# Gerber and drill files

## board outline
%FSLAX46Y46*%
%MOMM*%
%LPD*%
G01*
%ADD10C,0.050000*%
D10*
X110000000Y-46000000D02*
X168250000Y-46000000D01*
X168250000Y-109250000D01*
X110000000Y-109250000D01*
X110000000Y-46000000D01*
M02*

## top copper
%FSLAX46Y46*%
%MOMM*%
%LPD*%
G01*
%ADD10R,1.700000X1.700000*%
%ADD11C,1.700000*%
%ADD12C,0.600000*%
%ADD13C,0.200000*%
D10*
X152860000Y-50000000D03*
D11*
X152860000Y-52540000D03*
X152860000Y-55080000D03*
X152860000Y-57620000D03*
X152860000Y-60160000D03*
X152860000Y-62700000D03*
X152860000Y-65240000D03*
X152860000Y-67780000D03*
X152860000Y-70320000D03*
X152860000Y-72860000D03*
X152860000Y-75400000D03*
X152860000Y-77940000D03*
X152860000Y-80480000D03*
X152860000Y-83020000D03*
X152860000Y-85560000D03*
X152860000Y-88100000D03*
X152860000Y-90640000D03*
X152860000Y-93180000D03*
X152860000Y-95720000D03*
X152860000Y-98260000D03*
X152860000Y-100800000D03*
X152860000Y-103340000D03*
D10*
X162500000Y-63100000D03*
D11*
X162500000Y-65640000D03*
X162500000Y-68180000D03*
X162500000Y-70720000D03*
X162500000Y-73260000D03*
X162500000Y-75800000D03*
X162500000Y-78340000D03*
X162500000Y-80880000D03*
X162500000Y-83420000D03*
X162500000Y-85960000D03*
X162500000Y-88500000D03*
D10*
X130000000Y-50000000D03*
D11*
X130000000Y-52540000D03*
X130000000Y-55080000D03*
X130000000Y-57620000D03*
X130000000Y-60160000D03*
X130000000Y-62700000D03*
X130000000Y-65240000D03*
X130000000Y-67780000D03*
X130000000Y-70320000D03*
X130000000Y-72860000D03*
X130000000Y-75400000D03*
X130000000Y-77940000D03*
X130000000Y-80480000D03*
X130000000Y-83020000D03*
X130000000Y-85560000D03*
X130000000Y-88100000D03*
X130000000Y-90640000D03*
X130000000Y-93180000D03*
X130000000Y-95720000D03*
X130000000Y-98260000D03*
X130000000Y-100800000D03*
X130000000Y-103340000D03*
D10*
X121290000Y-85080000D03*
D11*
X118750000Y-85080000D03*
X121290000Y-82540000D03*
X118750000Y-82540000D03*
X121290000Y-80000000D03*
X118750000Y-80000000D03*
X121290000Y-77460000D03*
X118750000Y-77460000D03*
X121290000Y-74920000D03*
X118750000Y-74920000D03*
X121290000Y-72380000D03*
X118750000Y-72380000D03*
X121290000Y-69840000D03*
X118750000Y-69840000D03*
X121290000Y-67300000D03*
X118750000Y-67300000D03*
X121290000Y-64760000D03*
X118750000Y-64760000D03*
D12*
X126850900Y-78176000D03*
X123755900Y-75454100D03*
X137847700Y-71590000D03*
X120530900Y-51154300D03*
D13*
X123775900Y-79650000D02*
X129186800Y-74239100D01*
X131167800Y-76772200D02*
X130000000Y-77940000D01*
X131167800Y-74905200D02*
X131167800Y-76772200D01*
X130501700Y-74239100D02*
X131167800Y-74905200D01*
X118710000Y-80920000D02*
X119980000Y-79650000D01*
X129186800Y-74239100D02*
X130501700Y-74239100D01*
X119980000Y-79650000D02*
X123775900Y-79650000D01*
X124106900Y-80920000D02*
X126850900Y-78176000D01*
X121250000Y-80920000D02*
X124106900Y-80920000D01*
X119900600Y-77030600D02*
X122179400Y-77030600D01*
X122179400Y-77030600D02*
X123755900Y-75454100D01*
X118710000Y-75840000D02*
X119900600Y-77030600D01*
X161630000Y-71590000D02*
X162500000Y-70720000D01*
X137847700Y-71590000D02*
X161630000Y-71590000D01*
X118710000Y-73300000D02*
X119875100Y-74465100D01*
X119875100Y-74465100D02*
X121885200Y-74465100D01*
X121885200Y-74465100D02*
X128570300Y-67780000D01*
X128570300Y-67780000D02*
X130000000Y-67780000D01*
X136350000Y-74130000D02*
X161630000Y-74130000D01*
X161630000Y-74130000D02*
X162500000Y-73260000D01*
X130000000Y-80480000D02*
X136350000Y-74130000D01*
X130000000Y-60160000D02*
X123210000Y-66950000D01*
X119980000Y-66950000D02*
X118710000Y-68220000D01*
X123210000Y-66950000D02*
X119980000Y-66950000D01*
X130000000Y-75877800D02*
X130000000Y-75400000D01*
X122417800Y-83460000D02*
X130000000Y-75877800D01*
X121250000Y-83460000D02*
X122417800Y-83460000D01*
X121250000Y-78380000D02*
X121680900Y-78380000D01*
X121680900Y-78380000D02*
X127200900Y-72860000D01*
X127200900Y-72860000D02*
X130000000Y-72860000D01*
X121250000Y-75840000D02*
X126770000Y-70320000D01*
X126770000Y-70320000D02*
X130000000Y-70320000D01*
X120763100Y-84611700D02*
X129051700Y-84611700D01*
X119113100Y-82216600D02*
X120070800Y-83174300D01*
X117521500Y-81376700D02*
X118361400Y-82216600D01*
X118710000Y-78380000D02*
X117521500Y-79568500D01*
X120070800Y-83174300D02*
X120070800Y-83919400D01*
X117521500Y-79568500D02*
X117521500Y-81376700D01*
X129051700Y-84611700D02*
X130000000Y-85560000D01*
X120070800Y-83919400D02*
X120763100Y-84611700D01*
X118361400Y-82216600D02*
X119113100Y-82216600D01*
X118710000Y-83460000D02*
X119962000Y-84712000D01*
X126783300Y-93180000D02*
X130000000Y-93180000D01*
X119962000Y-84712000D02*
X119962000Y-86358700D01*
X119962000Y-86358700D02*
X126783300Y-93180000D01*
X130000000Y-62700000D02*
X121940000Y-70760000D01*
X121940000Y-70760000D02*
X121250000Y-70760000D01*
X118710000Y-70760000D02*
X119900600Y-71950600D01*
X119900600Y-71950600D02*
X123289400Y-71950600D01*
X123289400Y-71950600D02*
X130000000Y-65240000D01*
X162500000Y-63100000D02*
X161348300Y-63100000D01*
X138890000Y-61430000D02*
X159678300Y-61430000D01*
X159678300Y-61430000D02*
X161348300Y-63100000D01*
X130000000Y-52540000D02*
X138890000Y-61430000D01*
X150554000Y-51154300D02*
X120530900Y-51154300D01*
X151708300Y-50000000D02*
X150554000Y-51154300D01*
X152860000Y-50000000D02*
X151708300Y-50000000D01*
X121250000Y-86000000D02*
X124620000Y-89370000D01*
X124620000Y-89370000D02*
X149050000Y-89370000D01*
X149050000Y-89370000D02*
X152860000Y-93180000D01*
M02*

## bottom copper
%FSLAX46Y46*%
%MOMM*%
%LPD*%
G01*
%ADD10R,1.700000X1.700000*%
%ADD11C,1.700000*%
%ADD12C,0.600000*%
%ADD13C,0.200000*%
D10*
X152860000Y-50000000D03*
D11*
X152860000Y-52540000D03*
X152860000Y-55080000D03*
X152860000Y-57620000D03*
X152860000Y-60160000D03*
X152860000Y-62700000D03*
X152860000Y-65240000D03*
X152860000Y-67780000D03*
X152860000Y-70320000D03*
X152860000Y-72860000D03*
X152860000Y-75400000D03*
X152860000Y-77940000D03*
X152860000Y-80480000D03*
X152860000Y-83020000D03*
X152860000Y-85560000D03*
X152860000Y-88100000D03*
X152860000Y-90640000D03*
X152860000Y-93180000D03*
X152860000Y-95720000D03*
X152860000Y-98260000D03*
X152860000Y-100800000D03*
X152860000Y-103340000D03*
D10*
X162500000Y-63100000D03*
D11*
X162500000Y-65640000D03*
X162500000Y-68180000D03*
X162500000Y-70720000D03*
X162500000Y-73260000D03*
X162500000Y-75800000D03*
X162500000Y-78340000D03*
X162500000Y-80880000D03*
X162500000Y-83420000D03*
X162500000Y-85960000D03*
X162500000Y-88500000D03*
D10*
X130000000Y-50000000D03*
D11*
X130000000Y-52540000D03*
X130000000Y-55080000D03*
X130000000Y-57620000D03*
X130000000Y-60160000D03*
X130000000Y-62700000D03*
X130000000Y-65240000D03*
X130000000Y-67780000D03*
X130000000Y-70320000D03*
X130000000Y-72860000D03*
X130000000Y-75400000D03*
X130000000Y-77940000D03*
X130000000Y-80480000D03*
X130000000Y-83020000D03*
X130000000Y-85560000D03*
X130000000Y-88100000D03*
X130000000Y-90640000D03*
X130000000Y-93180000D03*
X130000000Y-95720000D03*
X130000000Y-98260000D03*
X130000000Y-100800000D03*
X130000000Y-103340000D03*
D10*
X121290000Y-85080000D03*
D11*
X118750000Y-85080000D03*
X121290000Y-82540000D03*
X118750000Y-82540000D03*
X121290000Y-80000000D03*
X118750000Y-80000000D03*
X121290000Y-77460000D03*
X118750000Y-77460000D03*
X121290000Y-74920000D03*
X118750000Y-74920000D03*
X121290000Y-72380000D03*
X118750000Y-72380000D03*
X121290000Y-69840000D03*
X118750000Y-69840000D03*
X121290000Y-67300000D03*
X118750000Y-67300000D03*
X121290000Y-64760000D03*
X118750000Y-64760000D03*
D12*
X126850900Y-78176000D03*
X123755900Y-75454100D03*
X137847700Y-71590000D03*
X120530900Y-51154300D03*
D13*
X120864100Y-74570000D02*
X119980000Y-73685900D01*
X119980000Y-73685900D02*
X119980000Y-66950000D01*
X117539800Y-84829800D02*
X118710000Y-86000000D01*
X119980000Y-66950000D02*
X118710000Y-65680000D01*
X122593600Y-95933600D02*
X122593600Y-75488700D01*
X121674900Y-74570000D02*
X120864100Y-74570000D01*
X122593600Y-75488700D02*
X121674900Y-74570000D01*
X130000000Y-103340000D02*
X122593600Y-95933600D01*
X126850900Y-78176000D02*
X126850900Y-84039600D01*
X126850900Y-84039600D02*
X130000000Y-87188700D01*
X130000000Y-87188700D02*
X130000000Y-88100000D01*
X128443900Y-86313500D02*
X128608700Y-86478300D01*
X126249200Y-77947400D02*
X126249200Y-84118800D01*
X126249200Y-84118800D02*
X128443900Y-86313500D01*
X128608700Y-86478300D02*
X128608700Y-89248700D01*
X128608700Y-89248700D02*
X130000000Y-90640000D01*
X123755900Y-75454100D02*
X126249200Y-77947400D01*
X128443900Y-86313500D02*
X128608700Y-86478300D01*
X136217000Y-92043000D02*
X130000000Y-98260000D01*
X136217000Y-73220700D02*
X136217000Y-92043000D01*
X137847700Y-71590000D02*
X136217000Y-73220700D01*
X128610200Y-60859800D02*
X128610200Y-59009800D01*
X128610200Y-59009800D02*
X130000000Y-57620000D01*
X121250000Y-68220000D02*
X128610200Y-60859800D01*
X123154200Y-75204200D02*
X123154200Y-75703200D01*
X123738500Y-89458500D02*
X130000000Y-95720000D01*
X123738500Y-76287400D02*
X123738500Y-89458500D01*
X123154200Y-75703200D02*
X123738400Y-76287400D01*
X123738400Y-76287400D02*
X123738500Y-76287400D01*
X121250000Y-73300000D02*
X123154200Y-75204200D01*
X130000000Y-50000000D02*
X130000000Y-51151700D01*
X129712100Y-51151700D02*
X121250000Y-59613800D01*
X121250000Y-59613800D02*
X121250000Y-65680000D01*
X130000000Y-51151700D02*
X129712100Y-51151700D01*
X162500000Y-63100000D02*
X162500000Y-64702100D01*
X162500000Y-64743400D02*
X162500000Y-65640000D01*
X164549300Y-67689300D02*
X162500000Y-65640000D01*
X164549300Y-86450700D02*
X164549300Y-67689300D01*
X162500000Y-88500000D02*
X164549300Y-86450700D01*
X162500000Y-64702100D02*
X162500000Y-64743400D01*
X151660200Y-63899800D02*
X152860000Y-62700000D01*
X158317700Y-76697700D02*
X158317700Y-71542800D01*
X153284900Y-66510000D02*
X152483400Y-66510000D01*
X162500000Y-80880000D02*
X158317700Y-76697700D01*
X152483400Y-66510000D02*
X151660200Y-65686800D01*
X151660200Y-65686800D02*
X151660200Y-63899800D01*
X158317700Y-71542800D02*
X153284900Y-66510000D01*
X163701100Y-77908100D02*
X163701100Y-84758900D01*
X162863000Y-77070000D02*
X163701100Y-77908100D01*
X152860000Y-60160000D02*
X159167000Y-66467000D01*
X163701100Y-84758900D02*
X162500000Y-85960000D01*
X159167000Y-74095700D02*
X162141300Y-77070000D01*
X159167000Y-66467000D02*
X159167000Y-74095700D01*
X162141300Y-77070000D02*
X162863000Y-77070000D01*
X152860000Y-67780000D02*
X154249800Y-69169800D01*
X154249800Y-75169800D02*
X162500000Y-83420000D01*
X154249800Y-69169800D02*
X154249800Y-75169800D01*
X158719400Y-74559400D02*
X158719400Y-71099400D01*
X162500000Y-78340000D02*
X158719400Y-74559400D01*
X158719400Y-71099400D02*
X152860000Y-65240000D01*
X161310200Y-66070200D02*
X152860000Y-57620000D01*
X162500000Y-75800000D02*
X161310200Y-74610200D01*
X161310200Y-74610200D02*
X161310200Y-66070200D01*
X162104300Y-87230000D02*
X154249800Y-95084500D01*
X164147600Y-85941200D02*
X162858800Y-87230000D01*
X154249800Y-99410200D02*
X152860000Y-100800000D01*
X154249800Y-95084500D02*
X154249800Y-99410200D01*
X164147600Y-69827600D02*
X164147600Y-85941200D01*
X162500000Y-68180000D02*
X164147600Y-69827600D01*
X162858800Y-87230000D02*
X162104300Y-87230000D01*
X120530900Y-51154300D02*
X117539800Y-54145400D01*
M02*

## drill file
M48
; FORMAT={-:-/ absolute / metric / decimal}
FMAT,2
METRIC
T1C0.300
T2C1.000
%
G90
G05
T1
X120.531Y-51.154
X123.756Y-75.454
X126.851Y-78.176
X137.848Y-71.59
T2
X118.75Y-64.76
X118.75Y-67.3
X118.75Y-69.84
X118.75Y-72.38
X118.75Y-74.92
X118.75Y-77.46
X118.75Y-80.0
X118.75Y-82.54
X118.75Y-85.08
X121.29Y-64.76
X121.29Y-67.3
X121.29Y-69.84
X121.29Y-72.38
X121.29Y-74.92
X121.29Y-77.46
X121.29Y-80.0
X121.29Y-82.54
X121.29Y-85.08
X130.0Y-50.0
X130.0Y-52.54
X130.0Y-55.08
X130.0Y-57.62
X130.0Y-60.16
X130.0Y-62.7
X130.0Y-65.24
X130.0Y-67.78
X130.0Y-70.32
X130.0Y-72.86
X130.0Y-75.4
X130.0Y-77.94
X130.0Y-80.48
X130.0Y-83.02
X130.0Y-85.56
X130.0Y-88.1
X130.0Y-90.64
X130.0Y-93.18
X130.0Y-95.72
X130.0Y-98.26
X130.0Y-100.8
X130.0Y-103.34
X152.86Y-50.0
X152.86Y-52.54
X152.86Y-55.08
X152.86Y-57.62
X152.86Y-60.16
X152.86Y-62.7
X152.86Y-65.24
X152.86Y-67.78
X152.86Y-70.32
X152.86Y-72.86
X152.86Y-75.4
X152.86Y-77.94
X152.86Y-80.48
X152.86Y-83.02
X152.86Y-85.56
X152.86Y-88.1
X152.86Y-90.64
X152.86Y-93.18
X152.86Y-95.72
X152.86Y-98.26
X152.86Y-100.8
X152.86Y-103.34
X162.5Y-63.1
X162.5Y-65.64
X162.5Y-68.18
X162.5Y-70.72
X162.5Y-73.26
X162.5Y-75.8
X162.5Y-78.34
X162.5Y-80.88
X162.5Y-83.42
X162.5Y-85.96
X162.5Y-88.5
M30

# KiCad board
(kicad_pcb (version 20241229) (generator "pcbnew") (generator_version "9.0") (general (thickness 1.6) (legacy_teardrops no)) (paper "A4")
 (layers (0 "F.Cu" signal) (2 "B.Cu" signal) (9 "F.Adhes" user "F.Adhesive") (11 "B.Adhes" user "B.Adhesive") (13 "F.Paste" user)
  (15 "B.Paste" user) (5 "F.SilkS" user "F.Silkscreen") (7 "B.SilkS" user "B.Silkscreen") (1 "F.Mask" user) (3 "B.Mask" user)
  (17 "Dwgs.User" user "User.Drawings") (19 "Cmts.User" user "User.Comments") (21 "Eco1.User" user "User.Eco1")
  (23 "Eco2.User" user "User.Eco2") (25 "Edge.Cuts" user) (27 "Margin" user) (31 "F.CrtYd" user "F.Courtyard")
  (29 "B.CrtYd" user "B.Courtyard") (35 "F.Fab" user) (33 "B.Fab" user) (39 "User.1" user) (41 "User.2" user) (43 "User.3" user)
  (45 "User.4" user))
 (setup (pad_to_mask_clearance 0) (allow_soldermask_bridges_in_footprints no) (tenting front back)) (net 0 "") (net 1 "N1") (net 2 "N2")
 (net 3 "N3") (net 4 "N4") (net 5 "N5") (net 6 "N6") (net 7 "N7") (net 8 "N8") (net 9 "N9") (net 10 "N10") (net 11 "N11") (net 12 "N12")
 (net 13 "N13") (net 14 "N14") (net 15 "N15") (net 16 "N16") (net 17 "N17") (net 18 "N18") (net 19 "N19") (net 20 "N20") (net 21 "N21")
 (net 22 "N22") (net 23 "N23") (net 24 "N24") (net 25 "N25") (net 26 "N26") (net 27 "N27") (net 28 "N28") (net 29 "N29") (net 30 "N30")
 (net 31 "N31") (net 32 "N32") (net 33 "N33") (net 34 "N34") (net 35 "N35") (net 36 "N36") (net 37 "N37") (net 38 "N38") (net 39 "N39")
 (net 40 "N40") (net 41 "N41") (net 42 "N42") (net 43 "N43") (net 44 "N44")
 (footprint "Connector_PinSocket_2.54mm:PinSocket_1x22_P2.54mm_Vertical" (layer "F.Cu") (at 152.86 50)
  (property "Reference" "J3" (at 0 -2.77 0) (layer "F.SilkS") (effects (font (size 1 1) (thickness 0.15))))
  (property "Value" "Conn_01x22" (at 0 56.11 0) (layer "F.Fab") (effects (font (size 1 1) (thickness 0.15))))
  (pad "1" thru_hole rect (at 0 0) (size 1.7 1.7) (drill 1) (layers "*.Cu" "*.Mask") (remove_unused_layers no) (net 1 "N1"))
  (pad "2" thru_hole circle (at 0 2.54) (size 1.7 1.7) (drill 1) (layers "*.Cu" "*.Mask") (remove_unused_layers no) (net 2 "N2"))
  (pad "3" thru_hole circle (at 0 5.08) (size 1.7 1.7) (drill 1) (layers "*.Cu" "*.Mask") (remove_unused_layers no) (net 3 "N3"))
  (pad "4" thru_hole circle (at 0 7.62) (size 1.7 1.7) (drill 1) (layers "*.Cu" "*.Mask") (remove_unused_layers no) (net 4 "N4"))
  (pad "5" thru_hole circle (at 0 10.16) (size 1.7 1.7) (drill 1) (layers "*.Cu" "*.Mask") (remove_unused_layers no) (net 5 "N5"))
  (pad "6" thru_hole circle (at 0 12.7) (size 1.7 1.7) (drill 1) (layers "*.Cu" "*.Mask") (remove_unused_layers no) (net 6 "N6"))
  (pad "7" thru_hole circle (at 0 15.24) (size 1.7 1.7) (drill 1) (layers "*.Cu" "*.Mask") (remove_unused_layers no) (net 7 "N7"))
  (pad "8" thru_hole circle (at 0 17.78) (size 1.7 1.7) (drill 1) (layers "*.Cu" "*.Mask") (remove_unused_layers no) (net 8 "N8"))
  (pad "9" thru_hole circle (at 0 20.32) (size 1.7 1.7) (drill 1) (layers "*.Cu" "*.Mask") (remove_unused_layers no) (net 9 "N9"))
  (pad "10" thru_hole circle (at 0 22.86) (size 1.7 1.7) (drill 1) (layers "*.Cu" "*.Mask") (remove_unused_layers no) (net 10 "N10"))
  (pad "11" thru_hole circle (at 0 25.4) (size 1.7 1.7) (drill 1) (layers "*.Cu" "*.Mask") (remove_unused_layers no) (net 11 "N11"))
  (pad "12" thru_hole circle (at 0 27.94) (size 1.7 1.7) (drill 1) (layers "*.Cu" "*.Mask") (remove_unused_layers no) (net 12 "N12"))
  (pad "13" thru_hole circle (at 0 30.48) (size 1.7 1.7) (drill 1) (layers "*.Cu" "*.Mask") (remove_unused_layers no) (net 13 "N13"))
  (pad "14" thru_hole circle (at 0 33.02) (size 1.7 1.7) (drill 1) (layers "*.Cu" "*.Mask") (remove_unused_layers no) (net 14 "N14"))
  (pad "15" thru_hole circle (at 0 35.56) (size 1.7 1.7) (drill 1) (layers "*.Cu" "*.Mask") (remove_unused_layers no) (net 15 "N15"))
  (pad "16" thru_hole circle (at 0 38.1) (size 1.7 1.7) (drill 1) (layers "*.Cu" "*.Mask") (remove_unused_layers no) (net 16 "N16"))
  (pad "17" thru_hole circle (at 0 40.64) (size 1.7 1.7) (drill 1) (layers "*.Cu" "*.Mask") (remove_unused_layers no) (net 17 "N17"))
  (pad "18" thru_hole circle (at 0 43.18) (size 1.7 1.7) (drill 1) (layers "*.Cu" "*.Mask") (remove_unused_layers no) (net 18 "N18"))
  (pad "19" thru_hole circle (at 0 45.72) (size 1.7 1.7) (drill 1) (layers "*.Cu" "*.Mask") (remove_unused_layers no) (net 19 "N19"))
  (pad "20" thru_hole circle (at 0 48.26) (size 1.7 1.7) (drill 1) (layers "*.Cu" "*.Mask") (remove_unused_layers no) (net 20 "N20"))
  (pad "21" thru_hole circle (at 0 50.8) (size 1.7 1.7) (drill 1) (layers "*.Cu" "*.Mask") (remove_unused_layers no) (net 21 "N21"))
  (pad "22" thru_hole circle (at 0 53.34) (size 1.7 1.7) (drill 1) (layers "*.Cu" "*.Mask") (remove_unused_layers no) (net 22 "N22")))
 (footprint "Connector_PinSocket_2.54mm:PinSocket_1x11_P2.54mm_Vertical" (layer "F.Cu") (at 162.5 63.1)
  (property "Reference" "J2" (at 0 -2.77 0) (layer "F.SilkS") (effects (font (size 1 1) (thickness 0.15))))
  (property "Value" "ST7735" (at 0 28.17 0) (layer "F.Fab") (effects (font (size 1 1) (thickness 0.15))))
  (pad "1" thru_hole rect (at 0 0) (size 1.7 1.7) (drill 1) (layers "*.Cu" "*.Mask") (remove_unused_layers no) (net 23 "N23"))
  (pad "2" thru_hole circle (at 0 2.54) (size 1.7 1.7) (drill 1) (layers "*.Cu" "*.Mask") (remove_unused_layers no) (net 23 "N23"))
  (pad "3" thru_hole circle (at 0 5.08) (size 1.7 1.7) (drill 1) (layers "*.Cu" "*.Mask") (remove_unused_layers no) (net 21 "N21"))
  (pad "4" thru_hole circle (at 0 7.62) (size 1.7 1.7) (drill 1) (layers "*.Cu" "*.Mask") (remove_unused_layers no) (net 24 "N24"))
  (pad "5" thru_hole circle (at 0 10.16) (size 1.7 1.7) (drill 1) (layers "*.Cu" "*.Mask") (remove_unused_layers no) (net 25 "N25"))
  (pad "6" thru_hole circle (at 0 12.7) (size 1.7 1.7) (drill 1) (layers "*.Cu" "*.Mask") (remove_unused_layers no) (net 4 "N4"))
  (pad "7" thru_hole circle (at 0 15.24) (size 1.7 1.7) (drill 1) (layers "*.Cu" "*.Mask") (remove_unused_layers no) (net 7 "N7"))
  (pad "8" thru_hole circle (at 0 17.78) (size 1.7 1.7) (drill 1) (layers "*.Cu" "*.Mask") (remove_unused_layers no) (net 6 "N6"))
  (pad "9" thru_hole circle (at 0 20.32) (size 1.7 1.7) (drill 1) (layers "*.Cu" "*.Mask") (remove_unused_layers no) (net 8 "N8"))
  (pad "10" thru_hole circle (at 0 22.86) (size 1.7 1.7) (drill 1) (layers "*.Cu" "*.Mask") (remove_unused_layers no) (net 5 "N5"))
  (pad "11" thru_hole circle (at 0 25.4) (size 1.7 1.7) (drill 1) (layers "*.Cu" "*.Mask") (remove_unused_layers no) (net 23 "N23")))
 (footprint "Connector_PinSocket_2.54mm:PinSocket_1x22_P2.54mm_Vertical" (layer "F.Cu") (at 130 50)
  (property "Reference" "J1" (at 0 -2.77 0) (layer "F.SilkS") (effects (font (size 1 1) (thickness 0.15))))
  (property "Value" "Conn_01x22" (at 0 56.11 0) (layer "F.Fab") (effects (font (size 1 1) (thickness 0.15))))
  (pad "1" thru_hole rect (at 0 0) (size 1.7 1.7) (drill 1) (layers "*.Cu" "*.Mask") (remove_unused_layers no) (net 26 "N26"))
  (pad "2" thru_hole circle (at 0 2.54) (size 1.7 1.7) (drill 1) (layers "*.Cu" "*.Mask") (remove_unused_layers no) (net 23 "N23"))
  (pad "3" thru_hole circle (at 0 5.08) (size 1.7 1.7) (drill 1) (layers "*.Cu" "*.Mask") (remove_unused_layers no) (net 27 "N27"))
  (pad "4" thru_hole circle (at 0 7.62) (size 1.7 1.7) (drill 1) (layers "*.Cu" "*.Mask") (remove_unused_layers no) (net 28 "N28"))
  (pad "5" thru_hole circle (at 0 10.16) (size 1.7 1.7) (drill 1) (layers "*.Cu" "*.Mask") (remove_unused_layers no) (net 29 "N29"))
  (pad "6" thru_hole circle (at 0 12.7) (size 1.7 1.7) (drill 1) (layers "*.Cu" "*.Mask") (remove_unused_layers no) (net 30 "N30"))
  (pad "7" thru_hole circle (at 0 15.24) (size 1.7 1.7) (drill 1) (layers "*.Cu" "*.Mask") (remove_unused_layers no) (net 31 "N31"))
  (pad "8" thru_hole circle (at 0 17.78) (size 1.7 1.7) (drill 1) (layers "*.Cu" "*.Mask") (remove_unused_layers no) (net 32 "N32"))
  (pad "9" thru_hole circle (at 0 20.32) (size 1.7 1.7) (drill 1) (layers "*.Cu" "*.Mask") (remove_unused_layers no) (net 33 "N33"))
  (pad "10" thru_hole circle (at 0 22.86) (size 1.7 1.7) (drill 1) (layers "*.Cu" "*.Mask") (remove_unused_layers no) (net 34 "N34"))
  (pad "11" thru_hole circle (at 0 25.4) (size 1.7 1.7) (drill 1) (layers "*.Cu" "*.Mask") (remove_unused_layers no) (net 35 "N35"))
  (pad "12" thru_hole circle (at 0 27.94) (size 1.7 1.7) (drill 1) (layers "*.Cu" "*.Mask") (remove_unused_layers no) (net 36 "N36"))
  (pad "13" thru_hole circle (at 0 30.48) (size 1.7 1.7) (drill 1) (layers "*.Cu" "*.Mask") (remove_unused_layers no) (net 25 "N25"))
  (pad "14" thru_hole circle (at 0 33.02) (size 1.7 1.7) (drill 1) (layers "*.Cu" "*.Mask") (remove_unused_layers no) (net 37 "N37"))
  (pad "15" thru_hole circle (at 0 35.56) (size 1.7 1.7) (drill 1) (layers "*.Cu" "*.Mask") (remove_unused_layers no) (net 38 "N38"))
  (pad "16" thru_hole circle (at 0 38.1) (size 1.7 1.7) (drill 1) (layers "*.Cu" "*.Mask") (remove_unused_layers no) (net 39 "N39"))
  (pad "17" thru_hole circle (at 0 40.64) (size 1.7 1.7) (drill 1) (layers "*.Cu" "*.Mask") (remove_unused_layers no) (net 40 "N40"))
  (pad "18" thru_hole circle (at 0 43.18) (size 1.7 1.7) (drill 1) (layers "*.Cu" "*.Mask") (remove_unused_layers no) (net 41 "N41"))
  (pad "19" thru_hole circle (at 0 45.72) (size 1.7 1.7) (drill 1) (layers "*.Cu" "*.Mask") (remove_unused_layers no) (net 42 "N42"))
  (pad "20" thru_hole circle (at 0 48.26) (size 1.7 1.7) (drill 1) (layers "*.Cu" "*.Mask") (remove_unused_layers no) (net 24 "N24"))
  (pad "21" thru_hole circle (at 0 50.8) (size 1.7 1.7) (drill 1) (layers "*.Cu" "*.Mask") (remove_unused_layers no) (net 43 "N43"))
  (pad "22" thru_hole circle (at 0 53.34) (size 1.7 1.7) (drill 1) (layers "*.Cu" "*.Mask") (remove_unused_layers no) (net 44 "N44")))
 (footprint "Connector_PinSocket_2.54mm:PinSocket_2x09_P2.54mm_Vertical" (layer "B.Cu") (at 121.29 85.08)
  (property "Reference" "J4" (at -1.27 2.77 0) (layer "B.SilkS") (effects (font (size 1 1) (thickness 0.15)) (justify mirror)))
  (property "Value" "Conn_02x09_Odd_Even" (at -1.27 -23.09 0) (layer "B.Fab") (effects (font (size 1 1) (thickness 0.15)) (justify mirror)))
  (pad "1" thru_hole rect (at 0 0) (size 1.7 1.7) (drill 1) (layers "*.Cu" "*.Mask") (remove_unused_layers no) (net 26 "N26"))
  (pad "2" thru_hole circle (at -2.54 0) (size 1.7 1.7) (drill 1) (layers "*.Cu" "*.Mask") (remove_unused_layers no) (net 44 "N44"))
  (pad "3" thru_hole circle (at 0 -2.54) (size 1.7 1.7) (drill 1) (layers "*.Cu" "*.Mask") (remove_unused_layers no) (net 28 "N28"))
  (pad "4" thru_hole circle (at -2.54 -2.54) (size 1.7 1.7) (drill 1) (layers "*.Cu" "*.Mask") (remove_unused_layers no) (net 29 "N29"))
  (pad "5" thru_hole circle (at 0 -5.08) (size 1.7 1.7) (drill 1) (layers "*.Cu" "*.Mask") (remove_unused_layers no) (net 30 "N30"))
  (pad "6" thru_hole circle (at -2.54 -5.08) (size 1.7 1.7) (drill 1) (layers "*.Cu" "*.Mask") (remove_unused_layers no) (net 31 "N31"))
  (pad "7" thru_hole circle (at 0 -7.62) (size 1.7 1.7) (drill 1) (layers "*.Cu" "*.Mask") (remove_unused_layers no) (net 42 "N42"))
  (pad "8" thru_hole circle (at -2.54 -7.62) (size 1.7 1.7) (drill 1) (layers "*.Cu" "*.Mask") (remove_unused_layers no) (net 32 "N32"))
  (pad "9" thru_hole circle (at 0 -10.16) (size 1.7 1.7) (drill 1) (layers "*.Cu" "*.Mask") (remove_unused_layers no) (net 33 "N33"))
  (pad "10" thru_hole circle (at -2.54 -10.16) (size 1.7 1.7) (drill 1) (layers "*.Cu" "*.Mask") (remove_unused_layers no) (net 40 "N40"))
  (pad "11" thru_hole circle (at 0 -12.7) (size 1.7 1.7) (drill 1) (layers "*.Cu" "*.Mask") (remove_unused_layers no) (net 34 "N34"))
  (pad "12" thru_hole circle (at -2.54 -12.7) (size 1.7 1.7) (drill 1) (layers "*.Cu" "*.Mask") (remove_unused_layers no) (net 38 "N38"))
  (pad "13" thru_hole circle (at 0 -15.24) (size 1.7 1.7) (drill 1) (layers "*.Cu" "*.Mask") (remove_unused_layers no) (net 39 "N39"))
  (pad "14" thru_hole circle (at -2.54 -15.24) (size 1.7 1.7) (drill 1) (layers "*.Cu" "*.Mask") (remove_unused_layers no) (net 36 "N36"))
  (pad "15" thru_hole circle (at 0 -17.78) (size 1.7 1.7) (drill 1) (layers "*.Cu" "*.Mask") (remove_unused_layers no) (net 35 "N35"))
  (pad "16" thru_hole circle (at -2.54 -17.78) (size 1.7 1.7) (drill 1) (layers "*.Cu" "*.Mask") (remove_unused_layers no) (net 41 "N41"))
  (pad "17" thru_hole circle (at 0 -20.32) (size 1.7 1.7) (drill 1) (layers "*.Cu" "*.Mask") (remove_unused_layers no) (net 18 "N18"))
  (pad "18" thru_hole circle (at -2.54 -20.32) (size 1.7 1.7) (drill 1) (layers "*.Cu" "*.Mask") (remove_unused_layers no) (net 1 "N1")))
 (gr_rect (start 110 46) (end 168.25 109.25) (stroke (width 0.05) (type default)) (fill no) (layer "Edge.Cuts"))
 (segment (start 123.7759 79.65) (end 129.1868 74.2391) (width 0.2) (layer "F.Cu") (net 36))
 (segment (start 131.1678 76.7722) (end 130 77.94) (width 0.2) (layer "F.Cu") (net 36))
 (segment (start 131.1678 74.9052) (end 131.1678 76.7722) (width 0.2) (layer "F.Cu") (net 36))
 (segment (start 130.5017 74.2391) (end 131.1678 74.9052) (width 0.2) (layer "F.Cu") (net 36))
 (segment (start 118.71 80.92) (end 119.98 79.65) (width 0.2) (layer "F.Cu") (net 36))
 (segment (start 129.1868 74.2391) (end 130.5017 74.2391) (width 0.2) (layer "F.Cu") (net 36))
 (segment (start 119.98 79.65) (end 123.7759 79.65) (width 0.2) (layer "F.Cu") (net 36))
 (segment (start 120.8641 74.57) (end 119.98 73.6859) (width 0.2) (layer "B.Cu") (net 44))
 (segment (start 119.98 73.6859) (end 119.98 66.95) (width 0.2) (layer "B.Cu") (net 44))
 (segment (start 117.5398 84.8298) (end 118.71 86) (width 0.2) (layer "B.Cu") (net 44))
 (segment (start 119.98 66.95) (end 118.71 65.68) (width 0.2) (layer "B.Cu") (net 44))
 (segment (start 122.5936 95.9336) (end 122.5936 75.4887) (width 0.2) (layer "B.Cu") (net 44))
 (segment (start 121.6749 74.57) (end 120.8641 74.57) (width 0.2) (layer "B.Cu") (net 44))
 (segment (start 122.5936 75.4887) (end 121.6749 74.57) (width 0.2) (layer "B.Cu") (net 44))
 (segment (start 130 103.34) (end 122.5936 95.9336) (width 0.2) (layer "B.Cu") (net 44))
 (segment (start 124.1069 80.92) (end 126.8509 78.176) (width 0.2) (layer "F.Cu") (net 39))
 (segment (start 121.25 80.92) (end 124.1069 80.92) (width 0.2) (layer "F.Cu") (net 39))
 (via (at 126.8509 78.176) (size 0.6) (drill 0.3) (layers "F.Cu" "B.Cu") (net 39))
 (segment (start 126.8509 78.176) (end 126.8509 84.0396) (width 0.2) (layer "B.Cu") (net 39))
 (segment (start 126.8509 84.0396) (end 130 87.1887) (width 0.2) (layer "B.Cu") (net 39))
 (segment (start 130 87.1887) (end 130 88.1) (width 0.2) (layer "B.Cu") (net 39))
 (segment (start 119.9006 77.0306) (end 122.1794 77.0306) (width 0.2) (layer "F.Cu") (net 40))
 (segment (start 122.1794 77.0306) (end 123.7559 75.4541) (width 0.2) (layer "F.Cu") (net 40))
 (segment (start 118.71 75.84) (end 119.9006 77.0306) (width 0.2) (layer "F.Cu") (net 40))
 (via (at 123.7559 75.4541) (size 0.6) (drill 0.3) (layers "F.Cu" "B.Cu") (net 40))
 (segment (start 128.4439 86.3135) (end 128.6087 86.4783) (width 0.2) (layer "B.Cu") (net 40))
 (segment (start 126.2492 77.9474) (end 126.2492 84.1188) (width 0.2) (layer "B.Cu") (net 40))
 (segment (start 126.2492 84.1188) (end 128.4439 86.3135) (width 0.2) (layer "B.Cu") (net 40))
 (segment (start 128.6087 86.4783) (end 128.6087 89.2487) (width 0.2) (layer "B.Cu") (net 40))
 (segment (start 128.6087 89.2487) (end 130 90.64) (width 0.2) (layer "B.Cu") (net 40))
 (segment (start 123.7559 75.4541) (end 126.2492 77.9474) (width 0.2) (layer "B.Cu") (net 40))
 (segment (start 128.4439 86.3135) (end 128.6087 86.4783) (width 0.2) (layer "B.Cu") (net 40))
 (segment (start 161.63 71.59) (end 162.5 70.72) (width 0.2) (layer "F.Cu") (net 24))
 (segment (start 137.8477 71.59) (end 161.63 71.59) (width 0.2) (layer "F.Cu") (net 24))
 (via (at 137.8477 71.59) (size 0.6) (drill 0.3) (layers "F.Cu" "B.Cu") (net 24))
 (segment (start 136.217 92.043) (end 130 98.26) (width 0.2) (layer "B.Cu") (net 24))
 (segment (start 136.217 73.2207) (end 136.217 92.043) (width 0.2) (layer "B.Cu") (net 24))
 (segment (start 137.8477 71.59) (end 136.217 73.2207) (width 0.2) (layer "B.Cu") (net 24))
 (segment (start 128.6102 60.8598) (end 128.6102 59.0098) (width 0.2) (layer "B.Cu") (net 28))
 (segment (start 128.6102 59.0098) (end 130 57.62) (width 0.2) (layer "B.Cu") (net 28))
 (segment (start 121.25 68.22) (end 128.6102 60.8598) (width 0.2) (layer "B.Cu") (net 28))
 (segment (start 118.71 73.3) (end 119.8751 74.4651) (width 0.2) (layer "F.Cu") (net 32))
 (segment (start 119.8751 74.4651) (end 121.8852 74.4651) (width 0.2) (layer "F.Cu") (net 32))
 (segment (start 121.8852 74.4651) (end 128.5703 67.78) (width 0.2) (layer "F.Cu") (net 32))
 (segment (start 128.5703 67.78) (end 130 67.78) (width 0.2) (layer "F.Cu") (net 32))
 (segment (start 136.35 74.13) (end 161.63 74.13) (width 0.2) (layer "F.Cu") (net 25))
 (segment (start 161.63 74.13) (end 162.5 73.26) (width 0.2) (layer "F.Cu") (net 25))
 (segment (start 130 80.48) (end 136.35 74.13) (width 0.2) (layer "F.Cu") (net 25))
 (segment (start 130 60.16) (end 123.21 66.95) (width 0.2) (layer "F.Cu") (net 29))
 (segment (start 119.98 66.95) (end 118.71 68.22) (width 0.2) (layer "F.Cu") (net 29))
 (segment (start 123.21 66.95) (end 119.98 66.95) (width 0.2) (layer "F.Cu") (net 29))
 (segment (start 123.1542 75.2042) (end 123.1542 75.7032) (width 0.2) (layer "B.Cu") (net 42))
 (segment (start 123.7385 89.4585) (end 130 95.72) (width 0.2) (layer "B.Cu") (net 42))
 (segment (start 123.7385 76.2874) (end 123.7385 89.4585) (width 0.2) (layer "B.Cu") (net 42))
 (segment (start 123.1542 75.7032) (end 123.7384 76.2874) (width 0.2) (layer "B.Cu") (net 42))
 (segment (start 123.7384 76.2874) (end 123.7385 76.2874) (width 0.2) (layer "B.Cu") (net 42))
 (segment (start 121.25 73.3) (end 123.1542 75.2042) (width 0.2) (layer "B.Cu") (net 42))
 (segment (start 130 75.8778) (end 130 75.4) (width 0.2) (layer "F.Cu") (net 35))
 (segment (start 122.4178 83.46) (end 130 75.8778) (width 0.2) (layer "F.Cu") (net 35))
 (segment (start 121.25 83.46) (end 122.4178 83.46) (width 0.2) (layer "F.Cu") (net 35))
 (segment (start 121.25 78.38) (end 121.6809 78.38) (width 0.2) (layer "F.Cu") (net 34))
 (segment (start 121.6809 78.38) (end 127.2009 72.86) (width 0.2) (layer "F.Cu") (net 34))
 (segment (start 127.2009 72.86) (end 130 72.86) (width 0.2) (layer "F.Cu") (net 34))
 (segment (start 121.25 75.84) (end 126.77 70.32) (width 0.2) (layer "F.Cu") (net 33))
 (segment (start 126.77 70.32) (end 130 70.32) (width 0.2) (layer "F.Cu") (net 33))
 (segment (start 130 50) (end 130 51.1517) (width 0.2) (layer "B.Cu") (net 26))
 (segment (start 129.7121 51.1517) (end 121.25 59.6138) (width 0.2) (layer "B.Cu") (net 26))
 (segment (start 121.25 59.6138) (end 121.25 65.68) (width 0.2) (layer "B.Cu") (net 26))
 (segment (start 130 51.1517) (end 129.7121 51.1517) (width 0.2) (layer "B.Cu") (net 26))
 (segment (start 120.7631 84.6117) (end 129.0517 84.6117) (width 0.2) (layer "F.Cu") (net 38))
 (segment (start 119.1131 82.2166) (end 120.0708 83.1743) (width 0.2) (layer "F.Cu") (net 38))
 (segment (start 117.5215 81.3767) (end 118.3614 82.2166) (width 0.2) (layer "F.Cu") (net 38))
 (segment (start 118.71 78.38) (end 117.5215 79.5685) (width 0.2) (layer "F.Cu") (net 38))
 (segment (start 120.0708 83.1743) (end 120.0708 83.9194) (width 0.2) (layer "F.Cu") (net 38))
 (segment (start 117.5215 79.5685) (end 117.5215 81.3767) (width 0.2) (layer "F.Cu") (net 38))
 (segment (start 129.0517 84.6117) (end 130 85.56) (width 0.2) (layer "F.Cu") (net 38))
 (segment (start 120.0708 83.9194) (end 120.7631 84.6117) (width 0.2) (layer "F.Cu") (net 38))
 (segment (start 118.3614 82.2166) (end 119.1131 82.2166) (width 0.2) (layer "F.Cu") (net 38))
 (segment (start 118.71 83.46) (end 119.962 84.712) (width 0.2) (layer "F.Cu") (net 41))
 (segment (start 126.7833 93.18) (end 130 93.18) (width 0.2) (layer "F.Cu") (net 41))
 (segment (start 119.962 84.712) (end 119.962 86.3587) (width 0.2) (layer "F.Cu") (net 41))
 (segment (start 119.962 86.3587) (end 126.7833 93.18) (width 0.2) (layer "F.Cu") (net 41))
 (segment (start 130 62.7) (end 121.94 70.76) (width 0.2) (layer "F.Cu") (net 30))
 (segment (start 121.94 70.76) (end 121.25 70.76) (width 0.2) (layer "F.Cu") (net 30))
 (segment (start 118.71 70.76) (end 119.9006 71.9506) (width 0.2) (layer "F.Cu") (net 31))
 (segment (start 119.9006 71.9506) (end 123.2894 71.9506) (width 0.2) (layer "F.Cu") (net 31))
 (segment (start 123.2894 71.9506) (end 130 65.24) (width 0.2) (layer "F.Cu") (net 31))
 (segment (start 162.5 63.1) (end 161.3483 63.1) (width 0.2) (layer "F.Cu") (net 23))
 (segment (start 138.89 61.43) (end 159.6783 61.43) (width 0.2) (layer "F.Cu") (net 23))
 (segment (start 159.6783 61.43) (end 161.3483 63.1) (width 0.2) (layer "F.Cu") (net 23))
 (segment (start 130 52.54) (end 138.89 61.43) (width 0.2) (layer "F.Cu") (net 23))
 (segment (start 162.5 63.1) (end 162.5 64.7021) (width 0.2) (layer "B.Cu") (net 23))
 (segment (start 162.5 64.7434) (end 162.5 65.64) (width 0.2) (layer "B.Cu") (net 23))
 (segment (start 164.5493 67.6893) (end 162.5 65.64) (width 0.2) (layer "B.Cu") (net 23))
 (segment (start 164.5493 86.4507) (end 164.5493 67.6893) (width 0.2) (layer "B.Cu") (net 23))
 (segment (start 162.5 88.5) (end 164.5493 86.4507) (width 0.2) (layer "B.Cu") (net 23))
 (segment (start 162.5 64.7021) (end 162.5 64.7434) (width 0.2) (layer "B.Cu") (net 23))
 (segment (start 151.6602 63.8998) (end 152.86 62.7) (width 0.2) (layer "B.Cu") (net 6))
 (segment (start 158.3177 76.6977) (end 158.3177 71.5428) (width 0.2) (layer "B.Cu") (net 6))
 (segment (start 153.2849 66.51) (end 152.4834 66.51) (width 0.2) (layer "B.Cu") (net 6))
 (segment (start 162.5 80.88) (end 158.3177 76.6977) (width 0.2) (layer "B.Cu") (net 6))
 (segment (start 152.4834 66.51) (end 151.6602 65.6868) (width 0.2) (layer "B.Cu") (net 6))
 (segment (start 151.6602 65.6868) (end 151.6602 63.8998) (width 0.2) (layer "B.Cu") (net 6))
 (segment (start 158.3177 71.5428) (end 153.2849 66.51) (width 0.2) (layer "B.Cu") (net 6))
 (segment (start 163.7011 77.9081) (end 163.7011 84.7589) (width 0.2) (layer "B.Cu") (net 5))
 (segment (start 162.863 77.07) (end 163.7011 77.9081) (width 0.2) (layer "B.Cu") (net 5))
 (segment (start 152.86 60.16) (end 159.167 66.467) (width 0.2) (layer "B.Cu") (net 5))
 (segment (start 163.7011 84.7589) (end 162.5 85.96) (width 0.2) (layer "B.Cu") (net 5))
 (segment (start 159.167 74.0957) (end 162.1413 77.07) (width 0.2) (layer "B.Cu") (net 5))
 (segment (start 159.167 66.467) (end 159.167 74.0957) (width 0.2) (layer "B.Cu") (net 5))
 (segment (start 162.1413 77.07) (end 162.863 77.07) (width 0.2) (layer "B.Cu") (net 5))
 (segment (start 152.86 67.78) (end 154.2498 69.1698) (width 0.2) (layer "B.Cu") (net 8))
 (segment (start 154.2498 75.1698) (end 162.5 83.42) (width 0.2) (layer "B.Cu") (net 8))
 (segment (start 154.2498 69.1698) (end 154.2498 75.1698) (width 0.2) (layer "B.Cu") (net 8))
 (segment (start 158.7194 74.5594) (end 158.7194 71.0994) (width 0.2) (layer "B.Cu") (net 7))
 (segment (start 162.5 78.34) (end 158.7194 74.5594) (width 0.2) (layer "B.Cu") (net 7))
 (segment (start 158.7194 71.0994) (end 152.86 65.24) (width 0.2) (layer "B.Cu") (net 7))
 (segment (start 161.3102 66.0702) (end 152.86 57.62) (width 0.2) (layer "B.Cu") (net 4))
 (segment (start 162.5 75.8) (end 161.3102 74.6102) (width 0.2) (layer "B.Cu") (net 4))
 (segment (start 161.3102 74.6102) (end 161.3102 66.0702) (width 0.2) (layer "B.Cu") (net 4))
 (segment (start 162.1043 87.23) (end 154.2498 95.0845) (width 0.2) (layer "B.Cu") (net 21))
 (segment (start 164.1476 85.9412) (end 162.8588 87.23) (width 0.2) (layer "B.Cu") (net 21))
 (segment (start 154.2498 99.4102) (end 152.86 100.8) (width 0.2) (layer "B.Cu") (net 21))
 (segment (start 154.2498 95.0845) (end 154.2498 99.4102) (width 0.2) (layer "B.Cu") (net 21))
 (segment (start 164.1476 69.8276) (end 164.1476 85.9412) (width 0.2) (layer "B.Cu") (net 21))
 (segment (start 162.5 68.18) (end 164.1476 69.8276) (width 0.2) (layer "B.Cu") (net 21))
 (segment (start 162.8588 87.23) (end 162.1043 87.23) (width 0.2) (layer "B.Cu") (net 21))
 (segment (start 150.554 51.1543) (end 120.5309 51.1543) (width 0.2) (layer "F.Cu") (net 1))
 (segment (start 151.7083 50) (end 150.554 51.1543) (width 0.2) (layer "F.Cu") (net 1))
 (segment (start 152.86 50) (end 151.7083 50) (width 0.2) (layer "F.Cu") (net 1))
 (via (at 120.5309 51.1543) (size 0.6) (drill 0.3) (layers "F.Cu" "B.Cu") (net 1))
 (segment (start 120.5309 51.1543) (end 117.5398 54.1454) (width 0.2) (layer "B.Cu") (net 1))
 (segment (start 121.25 86) (end 124.62 89.37) (width 0.2) (layer "F.Cu") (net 18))
 (segment (start 124.62 89.37) (end 149.05 89.37) (width 0.2) (layer "F.Cu") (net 18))
 (segment (start 149.05 89.37) (end 152.86 93.18) (width 0.2) (layer "F.Cu") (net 18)))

